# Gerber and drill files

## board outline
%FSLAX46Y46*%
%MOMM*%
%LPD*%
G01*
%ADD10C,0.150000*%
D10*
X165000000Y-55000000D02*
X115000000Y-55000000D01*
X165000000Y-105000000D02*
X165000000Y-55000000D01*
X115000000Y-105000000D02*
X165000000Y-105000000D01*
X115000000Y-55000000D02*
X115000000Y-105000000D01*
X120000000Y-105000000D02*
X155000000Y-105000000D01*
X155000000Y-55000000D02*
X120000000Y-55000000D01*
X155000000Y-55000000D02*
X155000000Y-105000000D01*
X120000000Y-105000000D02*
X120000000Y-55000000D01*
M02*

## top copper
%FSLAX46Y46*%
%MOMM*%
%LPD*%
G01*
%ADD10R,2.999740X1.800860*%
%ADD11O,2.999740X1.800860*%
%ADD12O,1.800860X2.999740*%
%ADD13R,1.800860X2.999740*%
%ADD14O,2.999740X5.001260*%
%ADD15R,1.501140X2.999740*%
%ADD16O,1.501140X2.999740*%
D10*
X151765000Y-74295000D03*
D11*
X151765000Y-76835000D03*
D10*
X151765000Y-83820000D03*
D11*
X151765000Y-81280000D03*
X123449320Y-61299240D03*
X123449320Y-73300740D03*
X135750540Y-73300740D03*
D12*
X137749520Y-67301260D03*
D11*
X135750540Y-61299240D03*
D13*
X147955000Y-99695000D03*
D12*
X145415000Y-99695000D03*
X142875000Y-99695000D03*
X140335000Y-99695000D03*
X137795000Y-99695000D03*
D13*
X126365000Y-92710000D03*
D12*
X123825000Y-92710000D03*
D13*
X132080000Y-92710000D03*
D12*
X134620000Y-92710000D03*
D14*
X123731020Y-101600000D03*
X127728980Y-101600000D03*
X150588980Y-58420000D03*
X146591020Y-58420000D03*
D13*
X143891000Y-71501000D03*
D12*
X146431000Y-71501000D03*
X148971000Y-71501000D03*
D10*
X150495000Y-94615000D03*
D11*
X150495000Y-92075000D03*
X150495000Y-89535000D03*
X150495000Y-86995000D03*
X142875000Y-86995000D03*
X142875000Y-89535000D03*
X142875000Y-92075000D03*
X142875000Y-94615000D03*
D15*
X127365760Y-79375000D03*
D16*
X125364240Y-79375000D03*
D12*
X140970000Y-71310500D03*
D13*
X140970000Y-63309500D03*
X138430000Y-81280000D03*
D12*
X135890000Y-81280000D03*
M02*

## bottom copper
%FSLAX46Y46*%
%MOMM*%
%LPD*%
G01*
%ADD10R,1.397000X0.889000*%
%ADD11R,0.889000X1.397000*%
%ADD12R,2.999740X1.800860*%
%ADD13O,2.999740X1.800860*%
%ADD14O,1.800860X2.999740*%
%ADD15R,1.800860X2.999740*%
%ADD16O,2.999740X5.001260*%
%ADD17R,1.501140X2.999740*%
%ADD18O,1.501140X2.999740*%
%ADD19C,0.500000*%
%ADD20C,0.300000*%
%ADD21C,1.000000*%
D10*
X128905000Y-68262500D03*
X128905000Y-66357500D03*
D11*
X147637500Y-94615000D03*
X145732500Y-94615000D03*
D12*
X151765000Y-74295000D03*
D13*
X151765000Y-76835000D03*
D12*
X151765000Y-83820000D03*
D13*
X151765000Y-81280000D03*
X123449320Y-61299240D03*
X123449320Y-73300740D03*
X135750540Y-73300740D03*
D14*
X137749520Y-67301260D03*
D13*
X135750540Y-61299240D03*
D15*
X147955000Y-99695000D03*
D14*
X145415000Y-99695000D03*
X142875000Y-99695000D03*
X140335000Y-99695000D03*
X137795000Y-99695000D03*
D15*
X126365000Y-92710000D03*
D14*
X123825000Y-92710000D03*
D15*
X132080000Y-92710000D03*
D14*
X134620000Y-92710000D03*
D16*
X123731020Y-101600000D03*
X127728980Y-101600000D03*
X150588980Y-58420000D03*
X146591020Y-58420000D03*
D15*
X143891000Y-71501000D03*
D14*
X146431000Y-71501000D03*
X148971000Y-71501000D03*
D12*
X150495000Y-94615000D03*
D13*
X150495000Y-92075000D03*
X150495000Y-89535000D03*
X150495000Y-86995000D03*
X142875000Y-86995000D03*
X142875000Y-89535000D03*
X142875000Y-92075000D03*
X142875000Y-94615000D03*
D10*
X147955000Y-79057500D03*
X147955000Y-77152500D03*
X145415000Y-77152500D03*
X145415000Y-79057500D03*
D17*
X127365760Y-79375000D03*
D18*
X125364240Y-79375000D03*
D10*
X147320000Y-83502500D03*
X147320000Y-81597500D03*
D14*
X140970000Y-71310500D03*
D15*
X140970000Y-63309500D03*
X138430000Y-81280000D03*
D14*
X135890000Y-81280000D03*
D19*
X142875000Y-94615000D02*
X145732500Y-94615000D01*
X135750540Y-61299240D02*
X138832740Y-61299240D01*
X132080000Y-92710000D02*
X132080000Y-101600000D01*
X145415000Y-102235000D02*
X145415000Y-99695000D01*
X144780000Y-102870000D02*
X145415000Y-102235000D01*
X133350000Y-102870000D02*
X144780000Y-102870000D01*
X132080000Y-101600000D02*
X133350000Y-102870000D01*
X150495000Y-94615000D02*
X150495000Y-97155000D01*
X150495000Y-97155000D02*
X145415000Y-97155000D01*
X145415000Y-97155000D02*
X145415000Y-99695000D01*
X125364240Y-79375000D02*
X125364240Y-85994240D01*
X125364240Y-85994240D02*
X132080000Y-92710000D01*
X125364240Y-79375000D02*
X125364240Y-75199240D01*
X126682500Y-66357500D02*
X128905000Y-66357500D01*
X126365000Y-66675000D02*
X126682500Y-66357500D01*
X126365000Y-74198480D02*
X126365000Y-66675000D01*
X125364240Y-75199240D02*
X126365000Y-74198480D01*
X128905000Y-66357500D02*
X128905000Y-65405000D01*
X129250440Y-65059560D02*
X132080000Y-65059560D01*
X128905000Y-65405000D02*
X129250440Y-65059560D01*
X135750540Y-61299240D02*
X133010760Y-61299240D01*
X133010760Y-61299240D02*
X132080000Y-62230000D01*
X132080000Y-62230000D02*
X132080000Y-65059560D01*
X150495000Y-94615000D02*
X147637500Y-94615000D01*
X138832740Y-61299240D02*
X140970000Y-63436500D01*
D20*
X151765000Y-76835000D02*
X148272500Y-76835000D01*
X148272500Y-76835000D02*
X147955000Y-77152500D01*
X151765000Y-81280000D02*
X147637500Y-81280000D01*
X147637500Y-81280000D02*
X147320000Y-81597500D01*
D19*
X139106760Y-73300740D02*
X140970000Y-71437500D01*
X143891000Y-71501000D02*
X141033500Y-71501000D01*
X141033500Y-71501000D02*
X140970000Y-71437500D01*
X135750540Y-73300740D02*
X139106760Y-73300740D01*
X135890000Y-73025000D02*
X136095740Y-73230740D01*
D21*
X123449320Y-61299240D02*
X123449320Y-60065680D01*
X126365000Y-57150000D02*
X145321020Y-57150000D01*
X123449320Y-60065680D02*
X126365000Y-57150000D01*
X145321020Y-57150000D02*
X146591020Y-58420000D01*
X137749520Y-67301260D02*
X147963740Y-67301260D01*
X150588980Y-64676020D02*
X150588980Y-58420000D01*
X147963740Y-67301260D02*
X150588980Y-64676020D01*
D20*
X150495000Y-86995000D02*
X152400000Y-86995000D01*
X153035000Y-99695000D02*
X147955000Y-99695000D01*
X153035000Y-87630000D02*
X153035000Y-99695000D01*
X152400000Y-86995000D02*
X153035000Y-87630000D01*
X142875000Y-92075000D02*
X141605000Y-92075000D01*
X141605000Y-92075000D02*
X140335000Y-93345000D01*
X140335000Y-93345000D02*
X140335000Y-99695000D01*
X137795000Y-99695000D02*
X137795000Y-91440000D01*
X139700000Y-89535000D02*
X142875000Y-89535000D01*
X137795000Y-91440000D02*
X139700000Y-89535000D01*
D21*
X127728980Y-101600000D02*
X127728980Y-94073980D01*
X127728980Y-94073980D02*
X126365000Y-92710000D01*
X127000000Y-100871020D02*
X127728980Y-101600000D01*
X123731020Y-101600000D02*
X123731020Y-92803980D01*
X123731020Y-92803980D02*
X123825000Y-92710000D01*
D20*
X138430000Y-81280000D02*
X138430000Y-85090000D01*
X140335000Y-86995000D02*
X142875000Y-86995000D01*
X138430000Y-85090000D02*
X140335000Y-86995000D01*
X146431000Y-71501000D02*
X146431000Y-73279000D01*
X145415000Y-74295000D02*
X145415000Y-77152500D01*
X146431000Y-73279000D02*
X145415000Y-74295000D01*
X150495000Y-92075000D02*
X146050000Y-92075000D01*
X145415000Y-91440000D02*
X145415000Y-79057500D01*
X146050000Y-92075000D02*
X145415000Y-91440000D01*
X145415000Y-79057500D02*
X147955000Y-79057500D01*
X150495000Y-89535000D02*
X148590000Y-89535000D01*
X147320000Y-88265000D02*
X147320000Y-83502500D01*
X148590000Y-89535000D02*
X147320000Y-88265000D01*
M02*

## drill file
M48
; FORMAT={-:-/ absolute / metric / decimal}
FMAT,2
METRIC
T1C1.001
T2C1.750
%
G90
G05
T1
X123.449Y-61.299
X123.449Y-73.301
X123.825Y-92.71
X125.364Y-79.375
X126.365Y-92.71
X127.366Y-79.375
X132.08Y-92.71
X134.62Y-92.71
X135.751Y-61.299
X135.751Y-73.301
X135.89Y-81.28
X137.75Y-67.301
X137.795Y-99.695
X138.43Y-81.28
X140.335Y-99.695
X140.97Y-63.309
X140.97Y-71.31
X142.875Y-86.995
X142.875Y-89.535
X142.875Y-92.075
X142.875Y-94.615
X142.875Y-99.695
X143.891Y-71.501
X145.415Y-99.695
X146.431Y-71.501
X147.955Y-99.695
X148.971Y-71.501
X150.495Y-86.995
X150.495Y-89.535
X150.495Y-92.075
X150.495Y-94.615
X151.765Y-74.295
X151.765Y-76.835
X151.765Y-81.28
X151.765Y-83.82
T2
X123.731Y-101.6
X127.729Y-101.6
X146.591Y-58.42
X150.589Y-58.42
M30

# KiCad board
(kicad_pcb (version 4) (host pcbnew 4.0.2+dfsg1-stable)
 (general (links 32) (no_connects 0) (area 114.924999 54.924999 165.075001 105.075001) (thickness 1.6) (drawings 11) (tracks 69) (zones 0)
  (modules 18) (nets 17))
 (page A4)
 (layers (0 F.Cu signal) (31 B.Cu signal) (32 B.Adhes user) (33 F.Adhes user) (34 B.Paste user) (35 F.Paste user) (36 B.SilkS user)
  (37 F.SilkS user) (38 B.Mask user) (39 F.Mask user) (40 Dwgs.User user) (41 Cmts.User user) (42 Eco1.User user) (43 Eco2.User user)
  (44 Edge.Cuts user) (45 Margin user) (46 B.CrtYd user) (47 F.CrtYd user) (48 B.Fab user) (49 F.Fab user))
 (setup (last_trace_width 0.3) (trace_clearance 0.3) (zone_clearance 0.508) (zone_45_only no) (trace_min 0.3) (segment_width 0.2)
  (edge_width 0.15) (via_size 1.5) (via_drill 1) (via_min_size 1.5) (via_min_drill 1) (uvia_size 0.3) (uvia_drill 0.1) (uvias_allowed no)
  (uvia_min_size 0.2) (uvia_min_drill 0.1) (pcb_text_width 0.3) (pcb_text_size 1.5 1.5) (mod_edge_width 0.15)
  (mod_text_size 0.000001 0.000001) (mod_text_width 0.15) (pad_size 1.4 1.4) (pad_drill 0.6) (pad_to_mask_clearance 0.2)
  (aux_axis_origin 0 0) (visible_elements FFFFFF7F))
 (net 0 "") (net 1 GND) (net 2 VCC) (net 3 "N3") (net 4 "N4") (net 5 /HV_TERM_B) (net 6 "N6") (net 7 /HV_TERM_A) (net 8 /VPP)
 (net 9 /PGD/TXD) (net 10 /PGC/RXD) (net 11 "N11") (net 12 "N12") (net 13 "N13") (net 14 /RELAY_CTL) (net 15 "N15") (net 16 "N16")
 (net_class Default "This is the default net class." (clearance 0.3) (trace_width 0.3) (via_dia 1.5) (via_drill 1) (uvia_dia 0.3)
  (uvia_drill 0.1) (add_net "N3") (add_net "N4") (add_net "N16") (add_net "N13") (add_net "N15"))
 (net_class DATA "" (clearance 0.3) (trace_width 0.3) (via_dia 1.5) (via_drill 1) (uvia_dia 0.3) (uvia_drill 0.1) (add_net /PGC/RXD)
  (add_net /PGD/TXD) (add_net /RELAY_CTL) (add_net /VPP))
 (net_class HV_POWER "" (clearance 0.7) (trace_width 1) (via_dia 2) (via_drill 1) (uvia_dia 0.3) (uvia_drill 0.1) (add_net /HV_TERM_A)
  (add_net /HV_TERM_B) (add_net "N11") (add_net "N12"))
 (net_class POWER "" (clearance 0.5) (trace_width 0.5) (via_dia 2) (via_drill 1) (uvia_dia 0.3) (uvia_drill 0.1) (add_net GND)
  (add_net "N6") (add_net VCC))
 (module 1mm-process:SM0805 (layer B.Cu) (at 128.905 67.31 90)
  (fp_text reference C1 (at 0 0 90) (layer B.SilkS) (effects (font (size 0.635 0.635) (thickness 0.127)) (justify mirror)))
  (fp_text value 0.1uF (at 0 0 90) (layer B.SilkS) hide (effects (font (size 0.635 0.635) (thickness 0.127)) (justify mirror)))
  (pad 1 smd rect (at -0.9525 0 90) (size 0.889 1.397) (layers B.Cu B.Paste B.Mask) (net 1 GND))
  (pad 2 smd rect (at 0.9525 0 90) (size 0.889 1.397) (layers B.Cu B.Paste B.Mask) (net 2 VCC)))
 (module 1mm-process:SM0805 (layer B.Cu) (at 146.685 94.615 180)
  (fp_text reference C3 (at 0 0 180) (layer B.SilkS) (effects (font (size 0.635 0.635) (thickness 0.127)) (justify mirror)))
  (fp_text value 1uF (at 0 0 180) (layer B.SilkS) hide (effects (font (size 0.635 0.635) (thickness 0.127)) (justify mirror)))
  (pad 1 smd rect (at -0.9525 0 180) (size 0.889 1.397) (layers B.Cu B.Paste B.Mask) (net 2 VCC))
  (pad 2 smd rect (at 0.9525 0 180) (size 0.889 1.397) (layers B.Cu B.Paste B.Mask) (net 1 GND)))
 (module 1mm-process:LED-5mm (layer F.Cu) (at 151.765 75.565 270)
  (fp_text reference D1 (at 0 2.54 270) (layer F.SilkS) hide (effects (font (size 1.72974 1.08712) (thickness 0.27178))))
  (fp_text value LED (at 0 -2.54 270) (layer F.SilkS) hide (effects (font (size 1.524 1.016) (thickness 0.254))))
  (pad 1 thru_hole rect (at -1.27 0 270) (size 1.80086 2.99974) (drill 1.00076) (layers *.Cu *.Mask F.SilkS) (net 1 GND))
  (pad 2 thru_hole oval (at 1.27 0 270) (size 1.80086 2.99974) (drill 1.00076) (layers *.Cu *.Mask F.SilkS) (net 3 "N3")))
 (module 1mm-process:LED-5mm (layer F.Cu) (at 151.765 82.55 90)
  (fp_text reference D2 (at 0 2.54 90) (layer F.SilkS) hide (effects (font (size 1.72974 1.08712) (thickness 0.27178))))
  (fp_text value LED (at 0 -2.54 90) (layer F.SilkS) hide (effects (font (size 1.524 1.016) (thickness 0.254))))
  (pad 1 thru_hole rect (at -1.27 0 90) (size 1.80086 2.99974) (drill 1.00076) (layers *.Cu *.Mask F.SilkS) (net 1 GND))
  (pad 2 thru_hole oval (at 1.27 0 90) (size 1.80086 2.99974) (drill 1.00076) (layers *.Cu *.Mask F.SilkS) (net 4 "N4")))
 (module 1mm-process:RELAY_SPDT (layer F.Cu) (at 120 75)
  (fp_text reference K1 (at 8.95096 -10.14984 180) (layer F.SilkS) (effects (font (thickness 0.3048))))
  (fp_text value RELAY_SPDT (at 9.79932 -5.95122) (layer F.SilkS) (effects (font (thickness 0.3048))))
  (pad 5 thru_hole oval (at 3.44932 -13.70076 90) (size 1.80086 2.99974) (drill 1.00076) (layers *.Cu *.Mask F.SilkS) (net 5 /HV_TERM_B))
  (pad 4 thru_hole oval (at 3.44932 -1.69926 90) (size 1.80086 2.99974) (drill 1.00076) (layers *.Cu *.Mask F.SilkS))
  (pad 2 thru_hole oval (at 15.75054 -1.69926 90) (size 1.80086 2.99974) (drill 1.00076) (layers *.Cu *.Mask F.SilkS) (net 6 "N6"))
  (pad 3 thru_hole oval (at 17.74952 -7.69874) (size 1.80086 2.99974) (drill 1.00076) (layers *.Cu *.Mask F.SilkS) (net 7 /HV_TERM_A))
  (pad 1 thru_hole oval (at 15.75054 -13.70076 90) (size 1.80086 2.99974) (drill 1.00076) (layers *.Cu *.Mask F.SilkS) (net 2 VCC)))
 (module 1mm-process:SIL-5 (layer F.Cu) (at 141.605 99.695 180)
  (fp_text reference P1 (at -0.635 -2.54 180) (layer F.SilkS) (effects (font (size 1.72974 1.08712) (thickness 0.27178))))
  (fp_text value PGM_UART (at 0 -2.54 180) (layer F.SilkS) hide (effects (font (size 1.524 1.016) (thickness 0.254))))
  (pad 1 thru_hole rect (at -6.35 0 180) (size 1.80086 2.99974) (drill 1.00076) (layers *.Cu *.Mask F.SilkS) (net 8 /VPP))
  (pad 2 thru_hole oval (at -3.81 0 180) (size 1.80086 2.99974) (drill 1.00076) (layers *.Cu *.Mask F.SilkS) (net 2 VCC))
  (pad 3 thru_hole oval (at -1.27 0 180) (size 1.80086 2.99974) (drill 1.00076) (layers *.Cu *.Mask F.SilkS) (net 1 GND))
  (pad 4 thru_hole oval (at 1.27 0 180) (size 1.80086 2.99974) (drill 1.00076) (layers *.Cu *.Mask F.SilkS) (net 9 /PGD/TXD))
  (pad 5 thru_hole oval (at 3.81 0 180) (size 1.80086 2.99974) (drill 1.00076) (layers *.Cu *.Mask F.SilkS) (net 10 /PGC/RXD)))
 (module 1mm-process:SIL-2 (layer F.Cu) (at 125.095 92.71 180)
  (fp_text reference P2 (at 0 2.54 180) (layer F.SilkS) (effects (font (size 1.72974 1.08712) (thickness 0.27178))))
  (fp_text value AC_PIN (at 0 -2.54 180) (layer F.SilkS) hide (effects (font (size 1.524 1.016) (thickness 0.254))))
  (pad 1 thru_hole rect (at -1.27 0 180) (size 1.80086 2.99974) (drill 1.00076) (layers *.Cu *.Mask F.SilkS) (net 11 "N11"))
  (pad 2 thru_hole oval (at 1.27 0 180) (size 1.80086 2.99974) (drill 1.00076) (layers *.Cu *.Mask F.SilkS) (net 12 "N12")))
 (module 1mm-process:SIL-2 (layer F.Cu) (at 133.35 92.71)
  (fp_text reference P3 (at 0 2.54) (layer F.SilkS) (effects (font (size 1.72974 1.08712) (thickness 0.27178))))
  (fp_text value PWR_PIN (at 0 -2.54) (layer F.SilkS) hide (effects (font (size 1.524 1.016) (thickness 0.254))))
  (pad 1 thru_hole rect (at -1.27 0) (size 1.80086 2.99974) (drill 1.00076) (layers *.Cu *.Mask F.SilkS) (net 2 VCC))
  (pad 2 thru_hole oval (at 1.27 0) (size 1.80086 2.99974) (drill 1.00076) (layers *.Cu *.Mask F.SilkS) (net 1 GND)))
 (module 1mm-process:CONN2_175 (layer F.Cu) (at 125.73 101.6)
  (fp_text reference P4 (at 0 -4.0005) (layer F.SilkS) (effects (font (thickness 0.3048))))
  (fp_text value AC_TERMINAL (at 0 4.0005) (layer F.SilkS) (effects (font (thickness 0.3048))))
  (pad 1 thru_hole oval (at -1.99898 0) (size 2.99974 5.00126) (drill 1.75006) (layers *.Cu *.Mask F.SilkS) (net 12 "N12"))
  (pad 2 thru_hole oval (at 1.99898 0) (size 2.99974 5.00126) (drill 1.75006) (layers *.Cu *.Mask F.SilkS) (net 11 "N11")))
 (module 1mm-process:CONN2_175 (layer F.Cu) (at 148.59 58.42 180)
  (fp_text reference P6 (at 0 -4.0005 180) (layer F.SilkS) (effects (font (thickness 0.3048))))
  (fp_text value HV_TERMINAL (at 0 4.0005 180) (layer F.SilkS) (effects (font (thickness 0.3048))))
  (pad 1 thru_hole oval (at -1.99898 0 180) (size 2.99974 5.00126) (drill 1.75006) (layers *.Cu *.Mask F.SilkS) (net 7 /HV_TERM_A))
  (pad 2 thru_hole oval (at 1.99898 0 180) (size 2.99974 5.00126) (drill 1.75006) (layers *.Cu *.Mask F.SilkS) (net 5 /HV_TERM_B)))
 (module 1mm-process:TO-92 (layer F.Cu) (at 146.431 71.501)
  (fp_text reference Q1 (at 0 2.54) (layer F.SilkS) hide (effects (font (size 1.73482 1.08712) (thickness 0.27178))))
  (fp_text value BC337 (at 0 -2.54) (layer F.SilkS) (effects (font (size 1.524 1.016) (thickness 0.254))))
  (pad 1 thru_hole rect (at -2.54 0) (size 1.80086 2.99974) (drill 1.00076) (layers *.Cu *.Mask F.SilkS) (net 6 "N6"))
  (pad 2 thru_hole oval (at 0 0) (size 1.80086 2.99974) (drill 1.00076) (layers *.Cu *.Mask F.SilkS) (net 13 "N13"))
  (pad 3 thru_hole oval (at 2.54 0) (size 1.80086 2.99974) (drill 1.00076) (layers *.Cu *.Mask F.SilkS) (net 1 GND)))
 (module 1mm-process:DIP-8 (layer F.Cu) (at 146.685 90.805 90)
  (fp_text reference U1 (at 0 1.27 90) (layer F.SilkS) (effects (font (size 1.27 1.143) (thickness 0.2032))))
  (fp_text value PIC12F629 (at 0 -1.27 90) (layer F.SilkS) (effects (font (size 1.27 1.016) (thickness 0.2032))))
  (pad 1 thru_hole rect (at -3.81 3.81 90) (size 1.80086 2.99974) (drill 1.00076) (layers *.Cu *.Mask F.SilkS) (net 2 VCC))
  (pad 2 thru_hole oval (at -1.27 3.81 90) (size 1.80086 2.99974) (drill 1.00076) (layers *.Cu *.Mask F.SilkS) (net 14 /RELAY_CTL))
  (pad 3 thru_hole oval (at 1.27 3.81 90) (size 1.80086 2.99974) (drill 1.00076) (layers *.Cu *.Mask F.SilkS) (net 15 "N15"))
  (pad 4 thru_hole oval (at 3.81 3.81 90) (size 1.80086 2.99974) (drill 1.00076) (layers *.Cu *.Mask F.SilkS) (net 8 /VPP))
  (pad 5 thru_hole oval (at 3.81 -3.81 90) (size 1.80086 2.99974) (drill 1.00076) (layers *.Cu *.Mask F.SilkS) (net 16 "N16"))
  (pad 6 thru_hole oval (at 1.27 -3.81 90) (size 1.80086 2.99974) (drill 1.00076) (layers *.Cu *.Mask F.SilkS) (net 10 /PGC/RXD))
  (pad 7 thru_hole oval (at -1.27 -3.81 90) (size 1.80086 2.99974) (drill 1.00076) (layers *.Cu *.Mask F.SilkS) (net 9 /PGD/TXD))
  (pad 8 thru_hole oval (at -3.81 -3.81 90) (size 1.80086 2.99974) (drill 1.00076) (layers *.Cu *.Mask F.SilkS) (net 1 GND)))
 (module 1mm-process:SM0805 (layer B.Cu) (at 147.955 78.105 90)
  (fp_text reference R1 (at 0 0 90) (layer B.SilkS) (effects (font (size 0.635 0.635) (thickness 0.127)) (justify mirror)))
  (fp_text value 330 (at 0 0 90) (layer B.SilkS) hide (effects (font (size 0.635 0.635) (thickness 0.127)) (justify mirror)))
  (pad 1 smd rect (at -0.9525 0 90) (size 0.889 1.397) (layers B.Cu B.Paste B.Mask) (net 14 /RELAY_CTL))
  (pad 2 smd rect (at 0.9525 0 90) (size 0.889 1.397) (layers B.Cu B.Paste B.Mask) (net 3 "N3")))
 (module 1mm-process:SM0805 (layer B.Cu) (at 145.415 78.105 270)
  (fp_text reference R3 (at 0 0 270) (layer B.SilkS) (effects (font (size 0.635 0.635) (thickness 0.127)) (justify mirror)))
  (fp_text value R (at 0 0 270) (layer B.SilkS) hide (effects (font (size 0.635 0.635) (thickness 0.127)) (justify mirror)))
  (pad 1 smd rect (at -0.9525 0 270) (size 0.889 1.397) (layers B.Cu B.Paste B.Mask) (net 13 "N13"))
  (pad 2 smd rect (at 0.9525 0 270) (size 0.889 1.397) (layers B.Cu B.Paste B.Mask) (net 14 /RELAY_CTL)))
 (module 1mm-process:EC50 (layer F.Cu) (at 126.365 79.375)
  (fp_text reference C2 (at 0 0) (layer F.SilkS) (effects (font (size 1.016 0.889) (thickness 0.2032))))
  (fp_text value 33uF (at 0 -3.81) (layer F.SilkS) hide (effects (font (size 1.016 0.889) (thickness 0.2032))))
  (pad 2 thru_hole rect (at 1.00076 0) (size 1.50114 2.99974) (drill 1.00076) (layers *.Cu *.Mask F.SilkS) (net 1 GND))
  (pad 1 thru_hole oval (at -1.00076 0) (size 1.50114 2.99974) (drill 1.00076) (layers *.Cu *.Mask F.SilkS) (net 2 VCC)))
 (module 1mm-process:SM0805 (layer B.Cu) (at 147.32 82.55 90)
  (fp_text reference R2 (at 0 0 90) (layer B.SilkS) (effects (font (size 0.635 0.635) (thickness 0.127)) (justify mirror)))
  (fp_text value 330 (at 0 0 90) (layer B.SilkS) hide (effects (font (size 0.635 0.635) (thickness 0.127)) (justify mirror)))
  (pad 1 smd rect (at -0.9525 0 90) (size 0.889 1.397) (layers B.Cu B.Paste B.Mask) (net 15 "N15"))
  (pad 2 smd rect (at 0.9525 0 90) (size 0.889 1.397) (layers B.Cu B.Paste B.Mask) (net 4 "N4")))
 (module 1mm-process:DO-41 (layer F.Cu) (at 140.97 67.31 90)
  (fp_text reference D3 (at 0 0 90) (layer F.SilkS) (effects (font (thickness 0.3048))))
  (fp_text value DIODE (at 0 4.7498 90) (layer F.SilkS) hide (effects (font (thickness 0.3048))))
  (pad 2 thru_hole oval (at -4.0005 0 180) (size 1.80086 2.99974) (drill 1.00076) (layers *.Cu *.Mask F.SilkS) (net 6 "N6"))
  (pad 1 thru_hole rect (at 4.0005 0 180) (size 1.80086 2.99974) (drill 1.00076) (layers *.Cu *.Mask F.SilkS) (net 2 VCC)))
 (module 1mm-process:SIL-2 (layer F.Cu) (at 137.16 81.28 180)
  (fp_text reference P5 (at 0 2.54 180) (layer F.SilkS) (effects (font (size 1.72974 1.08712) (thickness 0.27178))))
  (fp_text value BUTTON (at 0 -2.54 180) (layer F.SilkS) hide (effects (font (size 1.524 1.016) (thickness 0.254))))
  (pad 1 thru_hole rect (at -1.27 0 180) (size 1.80086 2.99974) (drill 1.00076) (layers *.Cu *.Mask F.SilkS) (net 16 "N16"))
  (pad 2 thru_hole oval (at 1.27 0 180) (size 1.80086 2.99974) (drill 1.00076) (layers *.Cu *.Mask F.SilkS) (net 1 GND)))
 (gr_line (start 165 55) (end 115 55) (angle 90) (layer Edge.Cuts) (width 0.15))
 (gr_line (start 165 105) (end 165 55) (angle 90) (layer Edge.Cuts) (width 0.15))
 (gr_line (start 115 105) (end 165 105) (angle 90) (layer Edge.Cuts) (width 0.15))
 (gr_line (start 115 55) (end 115 105) (angle 90) (layer Edge.Cuts) (width 0.15))
 (gr_line (start 120 105) (end 155 105) (angle 90) (layer Edge.Cuts) (width 0.15))
 (gr_line (start 155 55) (end 120 55) (angle 90) (layer Edge.Cuts) (width 0.15))
 (gr_line (start 155 55) (end 155 105) (angle 90) (layer Edge.Cuts) (width 0.15))
 (gr_line (start 120 105) (end 120 55) (angle 90) (layer Edge.Cuts) (width 0.15))
 (segment (start 142.875 94.615) (end 145.7325 94.615) (width 0.5) (layer B.Cu) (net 1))
 (segment (start 135.75054 61.29924) (end 138.83274 61.29924) (width 0.5) (layer B.Cu) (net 2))
 (segment (start 132.08 92.71) (end 132.08 101.6) (width 0.5) (layer B.Cu) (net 2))
 (segment (start 145.415 102.235) (end 145.415 99.695) (width 0.5) (layer B.Cu) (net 2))
 (segment (start 144.78 102.87) (end 145.415 102.235) (width 0.5) (layer B.Cu) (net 2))
 (segment (start 133.35 102.87) (end 144.78 102.87) (width 0.5) (layer B.Cu) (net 2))
 (segment (start 132.08 101.6) (end 133.35 102.87) (width 0.5) (layer B.Cu) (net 2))
 (segment (start 150.495 94.615) (end 150.495 97.155) (width 0.5) (layer B.Cu) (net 2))
 (segment (start 150.495 97.155) (end 145.415 97.155) (width 0.5) (layer B.Cu) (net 2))
 (segment (start 145.415 97.155) (end 145.415 99.695) (width 0.5) (layer B.Cu) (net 2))
 (segment (start 125.36424 79.375) (end 125.36424 85.99424) (width 0.5) (layer B.Cu) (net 2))
 (segment (start 125.36424 85.99424) (end 132.08 92.71) (width 0.5) (layer B.Cu) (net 2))
 (segment (start 125.36424 79.375) (end 125.36424 75.19924) (width 0.5) (layer B.Cu) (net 2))
 (segment (start 126.6825 66.3575) (end 128.905 66.3575) (width 0.5) (layer B.Cu) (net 2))
 (segment (start 126.365 66.675) (end 126.6825 66.3575) (width 0.5) (layer B.Cu) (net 2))
 (segment (start 126.365 74.19848) (end 126.365 66.675) (width 0.5) (layer B.Cu) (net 2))
 (segment (start 125.36424 75.19924) (end 126.365 74.19848) (width 0.5) (layer B.Cu) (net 2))
 (segment (start 128.905 66.3575) (end 128.905 65.405) (width 0.5) (layer B.Cu) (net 2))
 (segment (start 129.25044 65.05956) (end 132.08 65.05956) (width 0.5) (layer B.Cu) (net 2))
 (segment (start 128.905 65.405) (end 129.25044 65.05956) (width 0.5) (layer B.Cu) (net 2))
 (segment (start 135.75054 61.29924) (end 133.01076 61.29924) (width 0.5) (layer B.Cu) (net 2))
 (segment (start 133.01076 61.29924) (end 132.08 62.23) (width 0.5) (layer B.Cu) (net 2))
 (segment (start 132.08 62.23) (end 132.08 65.05956) (width 0.5) (layer B.Cu) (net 2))
 (segment (start 150.495 94.615) (end 147.6375 94.615) (width 0.5) (layer B.Cu) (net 2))
 (segment (start 138.83274 61.29924) (end 140.97 63.4365) (width 0.5) (layer B.Cu) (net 2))
 (segment (start 151.765 76.835) (end 148.2725 76.835) (width 0.3) (layer B.Cu) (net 3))
 (segment (start 148.2725 76.835) (end 147.955 77.1525) (width 0.3) (layer B.Cu) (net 3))
 (segment (start 151.765 81.28) (end 147.6375 81.28) (width 0.3) (layer B.Cu) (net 4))
 (segment (start 147.6375 81.28) (end 147.32 81.5975) (width 0.3) (layer B.Cu) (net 4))
 (segment (start 139.10676 73.30074) (end 140.97 71.4375) (width 0.5) (layer B.Cu) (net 6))
 (segment (start 143.891 71.501) (end 141.0335 71.501) (width 0.5) (layer B.Cu) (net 6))
 (segment (start 141.0335 71.501) (end 140.97 71.4375) (width 0.5) (layer B.Cu) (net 6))
 (segment (start 135.75054 73.30074) (end 139.10676 73.30074) (width 0.5) (layer B.Cu) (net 6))
 (segment (start 135.89 73.025) (end 136.09574 73.23074) (width 0.5) (layer B.Cu) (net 6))
 (segment (start 123.44932 61.29924) (end 123.44932 60.06568) (width 1) (layer B.Cu) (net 5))
 (segment (start 126.365 57.15) (end 145.32102 57.15) (width 1) (layer B.Cu) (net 5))
 (segment (start 123.44932 60.06568) (end 126.365 57.15) (width 1) (layer B.Cu) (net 5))
 (segment (start 145.32102 57.15) (end 146.59102 58.42) (width 1) (layer B.Cu) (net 5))
 (segment (start 137.74952 67.30126) (end 147.96374 67.30126) (width 1) (layer B.Cu) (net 7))
 (segment (start 150.58898 64.67602) (end 150.58898 58.42) (width 1) (layer B.Cu) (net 7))
 (segment (start 147.96374 67.30126) (end 150.58898 64.67602) (width 1) (layer B.Cu) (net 7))
 (segment (start 150.495 86.995) (end 152.4 86.995) (width 0.3) (layer B.Cu) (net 8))
 (segment (start 153.035 99.695) (end 147.955 99.695) (width 0.3) (layer B.Cu) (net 8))
 (segment (start 153.035 87.63) (end 153.035 99.695) (width 0.3) (layer B.Cu) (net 8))
 (segment (start 152.4 86.995) (end 153.035 87.63) (width 0.3) (layer B.Cu) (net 8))
 (segment (start 142.875 92.075) (end 141.605 92.075) (width 0.3) (layer B.Cu) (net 9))
 (segment (start 141.605 92.075) (end 140.335 93.345) (width 0.3) (layer B.Cu) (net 9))
 (segment (start 140.335 93.345) (end 140.335 99.695) (width 0.3) (layer B.Cu) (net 9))
 (segment (start 137.795 99.695) (end 137.795 91.44) (width 0.3) (layer B.Cu) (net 10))
 (segment (start 139.7 89.535) (end 142.875 89.535) (width 0.3) (layer B.Cu) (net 10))
 (segment (start 137.795 91.44) (end 139.7 89.535) (width 0.3) (layer B.Cu) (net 10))
 (segment (start 127.72898 101.6) (end 127.72898 94.07398) (width 1) (layer B.Cu) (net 11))
 (segment (start 127.72898 94.07398) (end 126.365 92.71) (width 1) (layer B.Cu) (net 11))
 (segment (start 127 100.87102) (end 127.72898 101.6) (width 1) (layer B.Cu) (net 11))
 (segment (start 123.73102 101.6) (end 123.73102 92.80398) (width 1) (layer B.Cu) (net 12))
 (segment (start 123.73102 92.80398) (end 123.825 92.71) (width 1) (layer B.Cu) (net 12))
 (segment (start 138.43 81.28) (end 138.43 85.09) (width 0.3) (layer B.Cu) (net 16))
 (segment (start 140.335 86.995) (end 142.875 86.995) (width 0.3) (layer B.Cu) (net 16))
 (segment (start 138.43 85.09) (end 140.335 86.995) (width 0.3) (layer B.Cu) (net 16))
 (segment (start 146.431 71.501) (end 146.431 73.279) (width 0.3) (layer B.Cu) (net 13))
 (segment (start 145.415 74.295) (end 145.415 77.1525) (width 0.3) (layer B.Cu) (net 13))
 (segment (start 146.431 73.279) (end 145.415 74.295) (width 0.3) (layer B.Cu) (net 13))
 (segment (start 150.495 92.075) (end 146.05 92.075) (width 0.3) (layer B.Cu) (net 14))
 (segment (start 145.415 91.44) (end 145.415 79.0575) (width 0.3) (layer B.Cu) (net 14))
 (segment (start 146.05 92.075) (end 145.415 91.44) (width 0.3) (layer B.Cu) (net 14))
 (segment (start 145.415 79.0575) (end 147.955 79.0575) (width 0.3) (layer B.Cu) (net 14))
 (segment (start 150.495 89.535) (end 148.59 89.535) (width 0.3) (layer B.Cu) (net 15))
 (segment (start 147.32 88.265) (end 147.32 83.5025) (width 0.3) (layer B.Cu) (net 15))
 (segment (start 148.59 89.535) (end 147.32 88.265) (width 0.3) (layer B.Cu) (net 15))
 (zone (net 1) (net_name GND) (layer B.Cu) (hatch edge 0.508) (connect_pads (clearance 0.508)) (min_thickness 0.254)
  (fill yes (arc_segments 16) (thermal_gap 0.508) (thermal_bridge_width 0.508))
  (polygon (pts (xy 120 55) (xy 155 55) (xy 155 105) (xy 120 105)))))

